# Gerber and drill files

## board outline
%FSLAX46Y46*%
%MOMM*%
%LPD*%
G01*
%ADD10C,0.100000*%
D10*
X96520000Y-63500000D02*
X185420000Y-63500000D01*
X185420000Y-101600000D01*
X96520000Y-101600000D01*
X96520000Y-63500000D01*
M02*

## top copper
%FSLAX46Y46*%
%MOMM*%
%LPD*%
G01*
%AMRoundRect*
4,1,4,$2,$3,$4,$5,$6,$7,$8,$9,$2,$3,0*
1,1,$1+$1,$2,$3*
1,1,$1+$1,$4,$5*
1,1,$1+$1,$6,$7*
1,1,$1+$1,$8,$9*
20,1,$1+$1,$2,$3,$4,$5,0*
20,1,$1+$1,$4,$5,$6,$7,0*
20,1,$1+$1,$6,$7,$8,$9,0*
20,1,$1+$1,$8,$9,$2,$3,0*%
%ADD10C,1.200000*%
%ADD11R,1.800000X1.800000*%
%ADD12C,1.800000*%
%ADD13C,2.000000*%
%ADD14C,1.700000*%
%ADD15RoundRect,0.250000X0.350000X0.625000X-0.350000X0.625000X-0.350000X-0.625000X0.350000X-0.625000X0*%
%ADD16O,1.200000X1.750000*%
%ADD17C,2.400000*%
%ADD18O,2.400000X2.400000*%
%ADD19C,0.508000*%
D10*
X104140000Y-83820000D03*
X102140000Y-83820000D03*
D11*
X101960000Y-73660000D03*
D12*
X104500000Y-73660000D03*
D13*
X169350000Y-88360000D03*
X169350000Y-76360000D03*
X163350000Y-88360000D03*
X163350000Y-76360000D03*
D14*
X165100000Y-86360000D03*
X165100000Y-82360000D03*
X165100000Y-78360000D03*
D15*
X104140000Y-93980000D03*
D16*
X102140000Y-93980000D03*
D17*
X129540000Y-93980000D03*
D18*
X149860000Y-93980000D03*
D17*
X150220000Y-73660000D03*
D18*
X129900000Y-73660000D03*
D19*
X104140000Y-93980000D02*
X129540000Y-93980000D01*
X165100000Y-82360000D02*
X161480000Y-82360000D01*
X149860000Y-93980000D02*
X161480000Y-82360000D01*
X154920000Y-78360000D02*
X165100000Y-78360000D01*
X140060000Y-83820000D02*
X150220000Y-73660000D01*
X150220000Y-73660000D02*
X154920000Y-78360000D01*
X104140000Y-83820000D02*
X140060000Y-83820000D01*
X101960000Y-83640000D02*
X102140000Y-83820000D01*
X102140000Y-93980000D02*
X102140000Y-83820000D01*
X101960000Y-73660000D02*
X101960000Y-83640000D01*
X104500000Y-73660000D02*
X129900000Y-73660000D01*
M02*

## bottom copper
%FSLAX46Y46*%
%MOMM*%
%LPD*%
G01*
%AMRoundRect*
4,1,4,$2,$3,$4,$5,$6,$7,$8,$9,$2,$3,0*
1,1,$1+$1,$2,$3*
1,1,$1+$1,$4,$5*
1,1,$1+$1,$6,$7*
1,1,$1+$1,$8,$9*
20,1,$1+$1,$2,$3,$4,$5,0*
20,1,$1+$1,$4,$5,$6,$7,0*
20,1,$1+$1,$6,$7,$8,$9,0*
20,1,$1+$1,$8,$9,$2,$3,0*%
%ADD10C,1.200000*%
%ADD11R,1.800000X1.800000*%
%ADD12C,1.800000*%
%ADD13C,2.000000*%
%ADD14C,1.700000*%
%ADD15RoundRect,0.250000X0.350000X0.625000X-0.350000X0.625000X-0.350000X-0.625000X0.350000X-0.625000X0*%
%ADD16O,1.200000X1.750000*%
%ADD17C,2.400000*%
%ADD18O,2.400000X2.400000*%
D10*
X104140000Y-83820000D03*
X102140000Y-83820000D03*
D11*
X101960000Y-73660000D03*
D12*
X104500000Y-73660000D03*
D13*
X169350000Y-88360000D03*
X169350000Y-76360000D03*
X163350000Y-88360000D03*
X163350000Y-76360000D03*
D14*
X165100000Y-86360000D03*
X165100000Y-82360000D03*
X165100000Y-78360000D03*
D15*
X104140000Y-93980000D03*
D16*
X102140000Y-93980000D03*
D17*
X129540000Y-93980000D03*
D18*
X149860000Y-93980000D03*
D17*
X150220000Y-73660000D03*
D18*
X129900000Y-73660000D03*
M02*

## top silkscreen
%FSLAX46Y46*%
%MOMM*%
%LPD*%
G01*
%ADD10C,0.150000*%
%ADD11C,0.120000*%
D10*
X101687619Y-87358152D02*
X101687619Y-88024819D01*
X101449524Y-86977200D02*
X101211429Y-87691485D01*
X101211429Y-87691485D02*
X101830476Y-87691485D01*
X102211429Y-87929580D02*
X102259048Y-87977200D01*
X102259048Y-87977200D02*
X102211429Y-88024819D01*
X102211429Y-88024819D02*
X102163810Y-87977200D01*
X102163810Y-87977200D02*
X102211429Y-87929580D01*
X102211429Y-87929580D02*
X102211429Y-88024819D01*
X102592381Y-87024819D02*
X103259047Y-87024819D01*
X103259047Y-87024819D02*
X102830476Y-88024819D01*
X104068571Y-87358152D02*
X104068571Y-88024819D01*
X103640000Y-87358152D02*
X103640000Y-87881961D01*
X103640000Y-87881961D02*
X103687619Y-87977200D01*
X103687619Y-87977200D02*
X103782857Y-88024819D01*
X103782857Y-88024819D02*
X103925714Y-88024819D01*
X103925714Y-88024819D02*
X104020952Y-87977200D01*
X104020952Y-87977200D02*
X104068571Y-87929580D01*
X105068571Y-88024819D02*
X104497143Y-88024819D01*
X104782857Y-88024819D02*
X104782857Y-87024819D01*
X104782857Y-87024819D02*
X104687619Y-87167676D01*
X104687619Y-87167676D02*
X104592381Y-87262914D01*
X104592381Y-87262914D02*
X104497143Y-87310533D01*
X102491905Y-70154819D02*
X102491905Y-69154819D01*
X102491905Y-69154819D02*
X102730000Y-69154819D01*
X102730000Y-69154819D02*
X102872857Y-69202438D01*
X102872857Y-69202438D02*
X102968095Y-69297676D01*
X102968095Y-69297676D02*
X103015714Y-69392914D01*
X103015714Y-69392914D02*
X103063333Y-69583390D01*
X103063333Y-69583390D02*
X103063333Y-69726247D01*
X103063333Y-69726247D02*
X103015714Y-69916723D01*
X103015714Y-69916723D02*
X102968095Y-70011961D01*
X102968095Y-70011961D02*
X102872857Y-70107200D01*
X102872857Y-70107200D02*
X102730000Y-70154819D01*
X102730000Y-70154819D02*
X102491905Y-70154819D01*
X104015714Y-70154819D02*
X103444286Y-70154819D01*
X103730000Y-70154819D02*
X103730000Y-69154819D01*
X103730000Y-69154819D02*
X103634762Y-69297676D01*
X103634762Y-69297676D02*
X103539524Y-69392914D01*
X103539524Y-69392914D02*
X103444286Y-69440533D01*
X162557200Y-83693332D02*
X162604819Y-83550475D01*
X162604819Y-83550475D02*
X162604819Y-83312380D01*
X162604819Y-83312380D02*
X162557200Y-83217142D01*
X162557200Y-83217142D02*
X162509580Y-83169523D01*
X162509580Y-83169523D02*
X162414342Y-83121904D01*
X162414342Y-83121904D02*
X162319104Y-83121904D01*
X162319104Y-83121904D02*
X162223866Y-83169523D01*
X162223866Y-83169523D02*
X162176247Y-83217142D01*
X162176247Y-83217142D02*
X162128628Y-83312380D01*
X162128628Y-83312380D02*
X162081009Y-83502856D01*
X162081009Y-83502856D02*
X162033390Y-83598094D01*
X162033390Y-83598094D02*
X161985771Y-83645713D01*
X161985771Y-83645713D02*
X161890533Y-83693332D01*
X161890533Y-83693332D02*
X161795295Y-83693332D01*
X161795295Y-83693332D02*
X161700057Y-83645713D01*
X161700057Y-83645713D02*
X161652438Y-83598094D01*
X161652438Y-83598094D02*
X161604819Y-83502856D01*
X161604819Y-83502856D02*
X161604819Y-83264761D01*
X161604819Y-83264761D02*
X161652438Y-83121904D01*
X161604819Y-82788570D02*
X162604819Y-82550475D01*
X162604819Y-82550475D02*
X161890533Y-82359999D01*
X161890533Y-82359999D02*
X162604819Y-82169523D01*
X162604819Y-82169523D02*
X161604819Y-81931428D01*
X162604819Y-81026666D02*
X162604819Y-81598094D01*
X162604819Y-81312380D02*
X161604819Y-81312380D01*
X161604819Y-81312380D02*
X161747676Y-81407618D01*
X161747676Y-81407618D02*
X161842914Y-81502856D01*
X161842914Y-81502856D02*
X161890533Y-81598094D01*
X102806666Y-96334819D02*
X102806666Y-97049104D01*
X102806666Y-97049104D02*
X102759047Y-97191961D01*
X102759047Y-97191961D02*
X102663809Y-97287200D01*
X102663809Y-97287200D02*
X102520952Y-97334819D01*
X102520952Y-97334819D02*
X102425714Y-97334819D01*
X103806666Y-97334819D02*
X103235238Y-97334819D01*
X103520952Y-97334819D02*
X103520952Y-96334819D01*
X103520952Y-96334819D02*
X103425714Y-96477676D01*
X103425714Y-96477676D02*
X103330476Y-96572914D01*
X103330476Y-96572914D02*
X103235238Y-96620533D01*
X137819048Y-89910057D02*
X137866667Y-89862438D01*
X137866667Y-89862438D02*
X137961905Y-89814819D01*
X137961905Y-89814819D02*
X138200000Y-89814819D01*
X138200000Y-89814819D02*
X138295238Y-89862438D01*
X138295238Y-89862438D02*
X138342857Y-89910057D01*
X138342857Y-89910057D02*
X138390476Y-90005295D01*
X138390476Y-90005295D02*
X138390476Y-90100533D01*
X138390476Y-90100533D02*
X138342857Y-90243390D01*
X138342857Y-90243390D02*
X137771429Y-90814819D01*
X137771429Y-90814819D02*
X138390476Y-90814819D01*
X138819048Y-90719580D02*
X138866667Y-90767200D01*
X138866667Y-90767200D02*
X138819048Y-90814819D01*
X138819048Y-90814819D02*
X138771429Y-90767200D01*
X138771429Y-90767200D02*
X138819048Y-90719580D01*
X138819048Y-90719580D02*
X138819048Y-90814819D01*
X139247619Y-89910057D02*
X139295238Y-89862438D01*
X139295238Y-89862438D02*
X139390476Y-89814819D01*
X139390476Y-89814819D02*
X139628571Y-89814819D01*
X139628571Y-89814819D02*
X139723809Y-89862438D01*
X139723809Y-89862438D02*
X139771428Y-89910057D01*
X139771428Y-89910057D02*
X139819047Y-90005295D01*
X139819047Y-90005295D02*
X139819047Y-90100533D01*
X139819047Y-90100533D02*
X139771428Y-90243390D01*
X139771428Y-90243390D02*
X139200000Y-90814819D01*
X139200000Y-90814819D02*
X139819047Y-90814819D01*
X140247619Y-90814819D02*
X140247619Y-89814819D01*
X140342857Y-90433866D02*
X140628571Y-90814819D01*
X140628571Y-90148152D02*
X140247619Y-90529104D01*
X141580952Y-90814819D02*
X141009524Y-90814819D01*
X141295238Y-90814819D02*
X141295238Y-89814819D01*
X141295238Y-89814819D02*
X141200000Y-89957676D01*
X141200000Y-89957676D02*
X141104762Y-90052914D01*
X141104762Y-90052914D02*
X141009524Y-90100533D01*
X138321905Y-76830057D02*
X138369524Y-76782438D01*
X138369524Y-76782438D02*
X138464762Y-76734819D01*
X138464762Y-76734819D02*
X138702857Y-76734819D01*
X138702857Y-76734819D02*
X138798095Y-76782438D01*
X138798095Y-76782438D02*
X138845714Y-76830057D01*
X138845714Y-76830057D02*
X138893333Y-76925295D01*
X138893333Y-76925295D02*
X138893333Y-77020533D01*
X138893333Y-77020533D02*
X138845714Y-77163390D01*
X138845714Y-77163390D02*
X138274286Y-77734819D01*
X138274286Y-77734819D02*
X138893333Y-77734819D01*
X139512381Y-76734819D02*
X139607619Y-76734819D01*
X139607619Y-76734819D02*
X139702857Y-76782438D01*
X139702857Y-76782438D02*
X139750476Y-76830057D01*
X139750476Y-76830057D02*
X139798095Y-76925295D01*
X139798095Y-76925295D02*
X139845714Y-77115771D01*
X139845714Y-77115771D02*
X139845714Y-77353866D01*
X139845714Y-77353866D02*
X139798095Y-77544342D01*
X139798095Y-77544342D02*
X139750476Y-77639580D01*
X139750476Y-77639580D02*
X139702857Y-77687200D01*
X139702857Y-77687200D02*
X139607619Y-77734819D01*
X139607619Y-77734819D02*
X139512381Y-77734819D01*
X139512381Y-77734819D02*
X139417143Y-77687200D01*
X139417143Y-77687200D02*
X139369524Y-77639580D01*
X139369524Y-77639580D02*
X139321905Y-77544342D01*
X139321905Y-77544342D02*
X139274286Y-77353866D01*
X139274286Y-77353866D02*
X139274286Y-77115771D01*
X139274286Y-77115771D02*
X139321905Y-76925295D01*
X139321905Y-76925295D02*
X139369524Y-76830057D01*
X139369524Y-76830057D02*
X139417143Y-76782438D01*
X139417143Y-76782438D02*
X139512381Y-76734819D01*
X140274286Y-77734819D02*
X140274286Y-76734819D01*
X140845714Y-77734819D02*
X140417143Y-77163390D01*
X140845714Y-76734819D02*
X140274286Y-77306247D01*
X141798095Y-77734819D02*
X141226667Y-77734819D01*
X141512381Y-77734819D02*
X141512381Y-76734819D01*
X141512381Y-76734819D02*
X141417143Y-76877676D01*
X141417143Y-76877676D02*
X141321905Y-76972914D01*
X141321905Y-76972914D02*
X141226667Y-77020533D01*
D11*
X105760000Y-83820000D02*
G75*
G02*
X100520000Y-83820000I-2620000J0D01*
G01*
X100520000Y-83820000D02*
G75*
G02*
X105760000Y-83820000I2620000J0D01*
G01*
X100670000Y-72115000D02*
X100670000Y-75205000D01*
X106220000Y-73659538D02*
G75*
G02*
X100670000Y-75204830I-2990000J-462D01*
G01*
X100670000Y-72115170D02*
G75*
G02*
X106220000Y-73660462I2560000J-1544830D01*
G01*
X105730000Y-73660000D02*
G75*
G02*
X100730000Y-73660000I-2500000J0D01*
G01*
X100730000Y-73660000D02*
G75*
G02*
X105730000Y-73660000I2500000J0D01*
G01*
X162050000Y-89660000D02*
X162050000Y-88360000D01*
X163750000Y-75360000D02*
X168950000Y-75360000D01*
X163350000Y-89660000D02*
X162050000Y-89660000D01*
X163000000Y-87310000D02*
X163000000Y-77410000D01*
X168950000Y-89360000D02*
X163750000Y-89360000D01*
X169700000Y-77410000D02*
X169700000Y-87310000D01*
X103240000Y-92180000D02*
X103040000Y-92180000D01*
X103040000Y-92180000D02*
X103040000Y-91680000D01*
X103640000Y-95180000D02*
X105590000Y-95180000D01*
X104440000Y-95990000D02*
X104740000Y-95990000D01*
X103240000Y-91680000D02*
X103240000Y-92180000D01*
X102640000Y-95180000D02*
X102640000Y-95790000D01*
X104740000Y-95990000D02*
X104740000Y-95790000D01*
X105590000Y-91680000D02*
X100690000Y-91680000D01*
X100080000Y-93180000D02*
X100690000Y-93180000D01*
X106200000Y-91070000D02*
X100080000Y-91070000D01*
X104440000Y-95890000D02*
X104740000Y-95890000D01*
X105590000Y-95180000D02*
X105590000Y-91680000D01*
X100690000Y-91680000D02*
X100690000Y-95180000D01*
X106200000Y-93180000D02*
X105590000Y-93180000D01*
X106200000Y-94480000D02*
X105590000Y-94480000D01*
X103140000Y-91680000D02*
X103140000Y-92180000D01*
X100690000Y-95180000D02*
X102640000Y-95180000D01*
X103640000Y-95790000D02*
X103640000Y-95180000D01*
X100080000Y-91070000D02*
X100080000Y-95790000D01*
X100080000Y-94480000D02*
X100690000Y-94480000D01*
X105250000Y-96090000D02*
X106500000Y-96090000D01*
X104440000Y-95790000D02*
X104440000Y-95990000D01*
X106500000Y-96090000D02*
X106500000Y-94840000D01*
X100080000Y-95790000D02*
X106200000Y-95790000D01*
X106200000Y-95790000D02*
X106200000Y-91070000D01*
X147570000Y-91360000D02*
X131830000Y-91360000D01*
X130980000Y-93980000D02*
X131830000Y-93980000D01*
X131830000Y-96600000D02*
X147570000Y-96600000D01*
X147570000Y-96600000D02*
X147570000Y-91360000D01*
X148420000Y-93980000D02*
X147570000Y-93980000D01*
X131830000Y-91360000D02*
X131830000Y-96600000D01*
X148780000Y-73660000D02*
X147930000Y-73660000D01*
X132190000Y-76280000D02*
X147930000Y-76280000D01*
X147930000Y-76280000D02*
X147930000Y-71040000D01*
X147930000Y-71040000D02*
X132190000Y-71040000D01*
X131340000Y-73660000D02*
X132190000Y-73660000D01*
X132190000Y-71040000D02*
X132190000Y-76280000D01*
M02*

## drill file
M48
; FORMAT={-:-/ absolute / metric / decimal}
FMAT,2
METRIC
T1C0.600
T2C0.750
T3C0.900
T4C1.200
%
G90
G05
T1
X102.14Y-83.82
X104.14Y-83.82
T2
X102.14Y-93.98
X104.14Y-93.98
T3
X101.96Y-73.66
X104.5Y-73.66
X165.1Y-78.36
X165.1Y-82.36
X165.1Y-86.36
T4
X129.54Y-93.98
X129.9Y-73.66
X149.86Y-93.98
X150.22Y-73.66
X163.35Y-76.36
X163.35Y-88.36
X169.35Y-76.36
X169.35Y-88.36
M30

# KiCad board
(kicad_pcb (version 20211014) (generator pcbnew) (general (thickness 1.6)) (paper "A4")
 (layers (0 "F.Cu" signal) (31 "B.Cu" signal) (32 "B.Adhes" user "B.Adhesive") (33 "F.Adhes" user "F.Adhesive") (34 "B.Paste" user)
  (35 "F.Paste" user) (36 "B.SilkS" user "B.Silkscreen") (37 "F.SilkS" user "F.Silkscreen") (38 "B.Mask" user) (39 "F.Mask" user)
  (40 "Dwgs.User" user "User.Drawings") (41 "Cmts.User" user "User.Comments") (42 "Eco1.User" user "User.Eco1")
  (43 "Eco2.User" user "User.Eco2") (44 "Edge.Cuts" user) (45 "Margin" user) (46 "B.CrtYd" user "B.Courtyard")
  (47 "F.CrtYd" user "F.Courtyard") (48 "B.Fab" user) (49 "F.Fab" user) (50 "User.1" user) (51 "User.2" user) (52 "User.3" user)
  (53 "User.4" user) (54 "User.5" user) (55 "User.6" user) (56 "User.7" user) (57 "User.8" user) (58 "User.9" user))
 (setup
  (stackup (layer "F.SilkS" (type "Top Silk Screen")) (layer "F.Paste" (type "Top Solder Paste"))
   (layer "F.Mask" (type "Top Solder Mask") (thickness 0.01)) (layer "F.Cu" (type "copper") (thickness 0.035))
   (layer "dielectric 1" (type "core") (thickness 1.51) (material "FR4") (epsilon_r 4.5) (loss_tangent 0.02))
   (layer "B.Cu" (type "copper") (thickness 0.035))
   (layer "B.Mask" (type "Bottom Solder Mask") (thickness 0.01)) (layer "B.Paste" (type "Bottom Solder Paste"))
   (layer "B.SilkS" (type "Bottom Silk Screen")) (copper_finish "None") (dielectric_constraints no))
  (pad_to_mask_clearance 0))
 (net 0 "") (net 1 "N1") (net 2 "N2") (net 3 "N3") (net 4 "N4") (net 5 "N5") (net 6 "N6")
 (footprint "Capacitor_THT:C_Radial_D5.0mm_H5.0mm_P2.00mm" (layer "F.Cu") (at 104.14 83.82 180)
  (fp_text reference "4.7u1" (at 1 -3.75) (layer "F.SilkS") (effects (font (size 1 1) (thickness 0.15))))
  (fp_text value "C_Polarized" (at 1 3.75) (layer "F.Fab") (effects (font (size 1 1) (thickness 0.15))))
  (fp_circle (center 1 0) (end 3.62 0) (layer "F.SilkS") (width 0.12) (fill none))
  (pad "1" thru_hole circle (at 0 0 180) (size 1.2 1.2) (drill 0.6) (layers *.Cu *.Mask) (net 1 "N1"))
  (pad "2" thru_hole circle (at 2 0 180) (size 1.2 1.2) (drill 0.6) (layers *.Cu *.Mask) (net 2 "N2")))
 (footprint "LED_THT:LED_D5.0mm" (layer "F.Cu") (at 101.96 73.66)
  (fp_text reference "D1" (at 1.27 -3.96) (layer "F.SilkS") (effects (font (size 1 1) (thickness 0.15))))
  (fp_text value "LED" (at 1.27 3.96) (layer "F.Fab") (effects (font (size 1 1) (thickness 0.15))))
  (fp_line (start -1.29 -1.545) (end -1.29 1.545) (layer "F.SilkS") (width 0.12))
  (fp_arc (start 4.26 -0.000462) (mid 2.072002 2.880433) (end -1.29 1.54483) (layer "F.SilkS") (width 0.12))
  (fp_arc (start -1.29 -1.54483) (mid 2.072002 -2.880433) (end 4.26 0.000462) (layer "F.SilkS") (width 0.12))
  (fp_circle (center 1.27 0) (end 3.77 0) (layer "F.SilkS") (width 0.12) (fill none))
  (pad "1" thru_hole rect (at 0 0) (size 1.8 1.8) (drill 0.9) (layers *.Cu *.Mask) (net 2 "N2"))
  (pad "2" thru_hole circle (at 2.54 0) (size 1.8 1.8) (drill 0.9) (layers *.Cu *.Mask) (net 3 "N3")))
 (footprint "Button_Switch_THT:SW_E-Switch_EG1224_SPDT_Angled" (layer "F.Cu") (at 165.1 86.36 90)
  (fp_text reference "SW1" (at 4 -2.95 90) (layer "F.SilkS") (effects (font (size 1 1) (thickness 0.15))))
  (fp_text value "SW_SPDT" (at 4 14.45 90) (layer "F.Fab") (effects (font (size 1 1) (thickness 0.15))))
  (fp_line (start -3.3 -3.05) (end -2 -3.05) (layer "F.SilkS") (width 0.12))
  (fp_line (start 11 -1.35) (end 11 3.85) (layer "F.SilkS") (width 0.12))
  (fp_line (start -3.3 -1.75) (end -3.3 -3.05) (layer "F.SilkS") (width 0.12))
  (fp_line (start -0.95 -2.1) (end 8.95 -2.1) (layer "F.SilkS") (width 0.12))
  (fp_line (start -3 3.85) (end -3 -1.35) (layer "F.SilkS") (width 0.12))
  (fp_line (start 8.95 4.6) (end -0.95 4.6) (layer "F.SilkS") (width 0.12))
  (pad "" thru_hole circle (at -2 4.25 90) (size 2 2) (drill 1.2) (layers *.Cu *.Mask))
  (pad "" thru_hole circle (at 10 4.25 90) (size 2 2) (drill 1.2) (layers *.Cu *.Mask))
  (pad "" thru_hole circle (at -2 -1.75 90) (size 2 2) (drill 1.2) (layers *.Cu *.Mask))
  (pad "" thru_hole circle (at 10 -1.75 90) (size 2 2) (drill 1.2) (layers *.Cu *.Mask))
  (pad "1" thru_hole circle (at 0 0 90) (size 1.7 1.7) (drill 0.9) (layers *.Cu *.Mask) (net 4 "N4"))
  (pad "2" thru_hole circle (at 4 0 90) (size 1.7 1.7) (drill 0.9) (layers *.Cu *.Mask) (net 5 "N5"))
  (pad "3" thru_hole circle (at 8 0 90) (size 1.7 1.7) (drill 0.9) (layers *.Cu *.Mask) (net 1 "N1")))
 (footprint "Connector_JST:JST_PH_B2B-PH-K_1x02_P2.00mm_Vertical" (layer "F.Cu") (at 104.14 93.98 180)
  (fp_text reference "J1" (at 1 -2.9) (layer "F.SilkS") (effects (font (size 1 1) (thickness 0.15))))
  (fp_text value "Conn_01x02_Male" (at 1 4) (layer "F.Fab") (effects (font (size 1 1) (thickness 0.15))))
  (fp_line (start 0.9 1.8) (end 1.1 1.8) (layer "F.SilkS") (width 0.12))
  (fp_line (start 1.1 1.8) (end 1.1 2.3) (layer "F.SilkS") (width 0.12))
  (fp_line (start 0.5 -1.2) (end -1.45 -1.2) (layer "F.SilkS") (width 0.12))
  (fp_line (start -0.3 -2.01) (end -0.6 -2.01) (layer "F.SilkS") (width 0.12))
  (fp_line (start 0.9 2.3) (end 0.9 1.8) (layer "F.SilkS") (width 0.12))
  (fp_line (start 1.5 -1.2) (end 1.5 -1.81) (layer "F.SilkS") (width 0.12))
  (fp_line (start -0.6 -2.01) (end -0.6 -1.81) (layer "F.SilkS") (width 0.12))
  (fp_line (start -1.45 2.3) (end 3.45 2.3) (layer "F.SilkS") (width 0.12))
  (fp_line (start 4.06 0.8) (end 3.45 0.8) (layer "F.SilkS") (width 0.12))
  (fp_line (start -2.06 2.91) (end 4.06 2.91) (layer "F.SilkS") (width 0.12))
  (fp_line (start -0.3 -1.91) (end -0.6 -1.91) (layer "F.SilkS") (width 0.12))
  (fp_line (start -1.45 -1.2) (end -1.45 2.3) (layer "F.SilkS") (width 0.12))
  (fp_line (start 3.45 2.3) (end 3.45 -1.2) (layer "F.SilkS") (width 0.12))
  (fp_line (start -2.06 0.8) (end -1.45 0.8) (layer "F.SilkS") (width 0.12))
  (fp_line (start -2.06 -0.5) (end -1.45 -0.5) (layer "F.SilkS") (width 0.12))
  (fp_line (start 1 2.3) (end 1 1.8) (layer "F.SilkS") (width 0.12))
  (fp_line (start 3.45 -1.2) (end 1.5 -1.2) (layer "F.SilkS") (width 0.12))
  (fp_line (start 0.5 -1.81) (end 0.5 -1.2) (layer "F.SilkS") (width 0.12))
  (fp_line (start 4.06 2.91) (end 4.06 -1.81) (layer "F.SilkS") (width 0.12))
  (fp_line (start 4.06 -0.5) (end 3.45 -0.5) (layer "F.SilkS") (width 0.12))
  (fp_line (start -1.11 -2.11) (end -2.36 -2.11) (layer "F.SilkS") (width 0.12))
  (fp_line (start -0.3 -1.81) (end -0.3 -2.01) (layer "F.SilkS") (width 0.12))
  (fp_line (start -2.36 -2.11) (end -2.36 -0.86) (layer "F.SilkS") (width 0.12))
  (fp_line (start 4.06 -1.81) (end -2.06 -1.81) (layer "F.SilkS") (width 0.12))
  (fp_line (start -2.06 -1.81) (end -2.06 2.91) (layer "F.SilkS") (width 0.12))
  (pad "1" thru_hole roundrect (at 0 0 180) (size 1.2 1.75) (drill 0.75) (layers *.Cu *.Mask) (roundrect_rratio 0.2083333333) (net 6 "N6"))
  (pad "2" thru_hole oval (at 2 0 180) (size 1.2 1.75) (drill 0.75) (layers *.Cu *.Mask) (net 2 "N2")))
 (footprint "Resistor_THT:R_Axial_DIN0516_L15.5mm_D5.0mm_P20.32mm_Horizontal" (layer "F.Cu") (at 129.54 93.98)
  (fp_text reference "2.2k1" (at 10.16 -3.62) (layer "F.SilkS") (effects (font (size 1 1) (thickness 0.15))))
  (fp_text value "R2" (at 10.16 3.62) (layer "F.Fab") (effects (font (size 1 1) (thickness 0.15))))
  (fp_line (start 18.03 -2.62) (end 2.29 -2.62) (layer "F.SilkS") (width 0.12))
  (fp_line (start 1.44 0) (end 2.29 0) (layer "F.SilkS") (width 0.12))
  (fp_line (start 2.29 2.62) (end 18.03 2.62) (layer "F.SilkS") (width 0.12))
  (fp_line (start 18.03 2.62) (end 18.03 -2.62) (layer "F.SilkS") (width 0.12))
  (fp_line (start 18.88 0) (end 18.03 0) (layer "F.SilkS") (width 0.12))
  (fp_line (start 2.29 -2.62) (end 2.29 2.62) (layer "F.SilkS") (width 0.12))
  (pad "1" thru_hole circle (at 0 0) (size 2.4 2.4) (drill 1.2) (layers *.Cu *.Mask) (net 6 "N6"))
  (pad "2" thru_hole oval (at 20.32 0) (size 2.4 2.4) (drill 1.2) (layers *.Cu *.Mask) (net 5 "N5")))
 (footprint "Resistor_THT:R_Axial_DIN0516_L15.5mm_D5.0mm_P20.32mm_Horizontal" (layer "F.Cu") (at 150.22 73.66 180)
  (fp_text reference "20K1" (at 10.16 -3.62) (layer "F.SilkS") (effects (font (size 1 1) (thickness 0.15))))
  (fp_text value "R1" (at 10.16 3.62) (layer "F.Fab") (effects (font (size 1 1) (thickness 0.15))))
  (fp_line (start 1.44 0) (end 2.29 0) (layer "F.SilkS") (width 0.12))
  (fp_line (start 18.03 -2.62) (end 2.29 -2.62) (layer "F.SilkS") (width 0.12))
  (fp_line (start 2.29 -2.62) (end 2.29 2.62) (layer "F.SilkS") (width 0.12))
  (fp_line (start 2.29 2.62) (end 18.03 2.62) (layer "F.SilkS") (width 0.12))
  (fp_line (start 18.88 0) (end 18.03 0) (layer "F.SilkS") (width 0.12))
  (fp_line (start 18.03 2.62) (end 18.03 -2.62) (layer "F.SilkS") (width 0.12))
  (pad "1" thru_hole circle (at 0 0 180) (size 2.4 2.4) (drill 1.2) (layers *.Cu *.Mask) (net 1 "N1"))
  (pad "2" thru_hole oval (at 20.32 0 180) (size 2.4 2.4) (drill 1.2) (layers *.Cu *.Mask) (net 3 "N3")))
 (gr_rect (start 185.42 101.6) (end 96.52 63.5) (layer "Edge.Cuts") (width 0.1) (fill none))
 (segment (start 104.14 93.98) (end 129.54 93.98) (width 0.508) (layer "F.Cu") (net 6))
 (segment (start 165.1 82.36) (end 161.48 82.36) (width 0.508) (layer "F.Cu") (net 5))
 (segment (start 149.86 93.98) (end 161.48 82.36) (width 0.508) (layer "F.Cu") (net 5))
 (segment (start 154.92 78.36) (end 165.1 78.36) (width 0.508) (layer "F.Cu") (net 1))
 (segment (start 140.06 83.82) (end 150.22 73.66) (width 0.508) (layer "F.Cu") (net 1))
 (segment (start 150.22 73.66) (end 154.92 78.36) (width 0.508) (layer "F.Cu") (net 1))
 (segment (start 104.14 83.82) (end 140.06 83.82) (width 0.508) (layer "F.Cu") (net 1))
 (segment (start 101.96 83.64) (end 102.14 83.82) (width 0.508) (layer "F.Cu") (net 2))
 (segment (start 102.14 93.98) (end 102.14 83.82) (width 0.508) (layer "F.Cu") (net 2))
 (segment (start 101.96 73.66) (end 101.96 83.64) (width 0.508) (layer "F.Cu") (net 2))
 (segment (start 104.5 73.66) (end 129.9 73.66) (width 0.508) (layer "F.Cu") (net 3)))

